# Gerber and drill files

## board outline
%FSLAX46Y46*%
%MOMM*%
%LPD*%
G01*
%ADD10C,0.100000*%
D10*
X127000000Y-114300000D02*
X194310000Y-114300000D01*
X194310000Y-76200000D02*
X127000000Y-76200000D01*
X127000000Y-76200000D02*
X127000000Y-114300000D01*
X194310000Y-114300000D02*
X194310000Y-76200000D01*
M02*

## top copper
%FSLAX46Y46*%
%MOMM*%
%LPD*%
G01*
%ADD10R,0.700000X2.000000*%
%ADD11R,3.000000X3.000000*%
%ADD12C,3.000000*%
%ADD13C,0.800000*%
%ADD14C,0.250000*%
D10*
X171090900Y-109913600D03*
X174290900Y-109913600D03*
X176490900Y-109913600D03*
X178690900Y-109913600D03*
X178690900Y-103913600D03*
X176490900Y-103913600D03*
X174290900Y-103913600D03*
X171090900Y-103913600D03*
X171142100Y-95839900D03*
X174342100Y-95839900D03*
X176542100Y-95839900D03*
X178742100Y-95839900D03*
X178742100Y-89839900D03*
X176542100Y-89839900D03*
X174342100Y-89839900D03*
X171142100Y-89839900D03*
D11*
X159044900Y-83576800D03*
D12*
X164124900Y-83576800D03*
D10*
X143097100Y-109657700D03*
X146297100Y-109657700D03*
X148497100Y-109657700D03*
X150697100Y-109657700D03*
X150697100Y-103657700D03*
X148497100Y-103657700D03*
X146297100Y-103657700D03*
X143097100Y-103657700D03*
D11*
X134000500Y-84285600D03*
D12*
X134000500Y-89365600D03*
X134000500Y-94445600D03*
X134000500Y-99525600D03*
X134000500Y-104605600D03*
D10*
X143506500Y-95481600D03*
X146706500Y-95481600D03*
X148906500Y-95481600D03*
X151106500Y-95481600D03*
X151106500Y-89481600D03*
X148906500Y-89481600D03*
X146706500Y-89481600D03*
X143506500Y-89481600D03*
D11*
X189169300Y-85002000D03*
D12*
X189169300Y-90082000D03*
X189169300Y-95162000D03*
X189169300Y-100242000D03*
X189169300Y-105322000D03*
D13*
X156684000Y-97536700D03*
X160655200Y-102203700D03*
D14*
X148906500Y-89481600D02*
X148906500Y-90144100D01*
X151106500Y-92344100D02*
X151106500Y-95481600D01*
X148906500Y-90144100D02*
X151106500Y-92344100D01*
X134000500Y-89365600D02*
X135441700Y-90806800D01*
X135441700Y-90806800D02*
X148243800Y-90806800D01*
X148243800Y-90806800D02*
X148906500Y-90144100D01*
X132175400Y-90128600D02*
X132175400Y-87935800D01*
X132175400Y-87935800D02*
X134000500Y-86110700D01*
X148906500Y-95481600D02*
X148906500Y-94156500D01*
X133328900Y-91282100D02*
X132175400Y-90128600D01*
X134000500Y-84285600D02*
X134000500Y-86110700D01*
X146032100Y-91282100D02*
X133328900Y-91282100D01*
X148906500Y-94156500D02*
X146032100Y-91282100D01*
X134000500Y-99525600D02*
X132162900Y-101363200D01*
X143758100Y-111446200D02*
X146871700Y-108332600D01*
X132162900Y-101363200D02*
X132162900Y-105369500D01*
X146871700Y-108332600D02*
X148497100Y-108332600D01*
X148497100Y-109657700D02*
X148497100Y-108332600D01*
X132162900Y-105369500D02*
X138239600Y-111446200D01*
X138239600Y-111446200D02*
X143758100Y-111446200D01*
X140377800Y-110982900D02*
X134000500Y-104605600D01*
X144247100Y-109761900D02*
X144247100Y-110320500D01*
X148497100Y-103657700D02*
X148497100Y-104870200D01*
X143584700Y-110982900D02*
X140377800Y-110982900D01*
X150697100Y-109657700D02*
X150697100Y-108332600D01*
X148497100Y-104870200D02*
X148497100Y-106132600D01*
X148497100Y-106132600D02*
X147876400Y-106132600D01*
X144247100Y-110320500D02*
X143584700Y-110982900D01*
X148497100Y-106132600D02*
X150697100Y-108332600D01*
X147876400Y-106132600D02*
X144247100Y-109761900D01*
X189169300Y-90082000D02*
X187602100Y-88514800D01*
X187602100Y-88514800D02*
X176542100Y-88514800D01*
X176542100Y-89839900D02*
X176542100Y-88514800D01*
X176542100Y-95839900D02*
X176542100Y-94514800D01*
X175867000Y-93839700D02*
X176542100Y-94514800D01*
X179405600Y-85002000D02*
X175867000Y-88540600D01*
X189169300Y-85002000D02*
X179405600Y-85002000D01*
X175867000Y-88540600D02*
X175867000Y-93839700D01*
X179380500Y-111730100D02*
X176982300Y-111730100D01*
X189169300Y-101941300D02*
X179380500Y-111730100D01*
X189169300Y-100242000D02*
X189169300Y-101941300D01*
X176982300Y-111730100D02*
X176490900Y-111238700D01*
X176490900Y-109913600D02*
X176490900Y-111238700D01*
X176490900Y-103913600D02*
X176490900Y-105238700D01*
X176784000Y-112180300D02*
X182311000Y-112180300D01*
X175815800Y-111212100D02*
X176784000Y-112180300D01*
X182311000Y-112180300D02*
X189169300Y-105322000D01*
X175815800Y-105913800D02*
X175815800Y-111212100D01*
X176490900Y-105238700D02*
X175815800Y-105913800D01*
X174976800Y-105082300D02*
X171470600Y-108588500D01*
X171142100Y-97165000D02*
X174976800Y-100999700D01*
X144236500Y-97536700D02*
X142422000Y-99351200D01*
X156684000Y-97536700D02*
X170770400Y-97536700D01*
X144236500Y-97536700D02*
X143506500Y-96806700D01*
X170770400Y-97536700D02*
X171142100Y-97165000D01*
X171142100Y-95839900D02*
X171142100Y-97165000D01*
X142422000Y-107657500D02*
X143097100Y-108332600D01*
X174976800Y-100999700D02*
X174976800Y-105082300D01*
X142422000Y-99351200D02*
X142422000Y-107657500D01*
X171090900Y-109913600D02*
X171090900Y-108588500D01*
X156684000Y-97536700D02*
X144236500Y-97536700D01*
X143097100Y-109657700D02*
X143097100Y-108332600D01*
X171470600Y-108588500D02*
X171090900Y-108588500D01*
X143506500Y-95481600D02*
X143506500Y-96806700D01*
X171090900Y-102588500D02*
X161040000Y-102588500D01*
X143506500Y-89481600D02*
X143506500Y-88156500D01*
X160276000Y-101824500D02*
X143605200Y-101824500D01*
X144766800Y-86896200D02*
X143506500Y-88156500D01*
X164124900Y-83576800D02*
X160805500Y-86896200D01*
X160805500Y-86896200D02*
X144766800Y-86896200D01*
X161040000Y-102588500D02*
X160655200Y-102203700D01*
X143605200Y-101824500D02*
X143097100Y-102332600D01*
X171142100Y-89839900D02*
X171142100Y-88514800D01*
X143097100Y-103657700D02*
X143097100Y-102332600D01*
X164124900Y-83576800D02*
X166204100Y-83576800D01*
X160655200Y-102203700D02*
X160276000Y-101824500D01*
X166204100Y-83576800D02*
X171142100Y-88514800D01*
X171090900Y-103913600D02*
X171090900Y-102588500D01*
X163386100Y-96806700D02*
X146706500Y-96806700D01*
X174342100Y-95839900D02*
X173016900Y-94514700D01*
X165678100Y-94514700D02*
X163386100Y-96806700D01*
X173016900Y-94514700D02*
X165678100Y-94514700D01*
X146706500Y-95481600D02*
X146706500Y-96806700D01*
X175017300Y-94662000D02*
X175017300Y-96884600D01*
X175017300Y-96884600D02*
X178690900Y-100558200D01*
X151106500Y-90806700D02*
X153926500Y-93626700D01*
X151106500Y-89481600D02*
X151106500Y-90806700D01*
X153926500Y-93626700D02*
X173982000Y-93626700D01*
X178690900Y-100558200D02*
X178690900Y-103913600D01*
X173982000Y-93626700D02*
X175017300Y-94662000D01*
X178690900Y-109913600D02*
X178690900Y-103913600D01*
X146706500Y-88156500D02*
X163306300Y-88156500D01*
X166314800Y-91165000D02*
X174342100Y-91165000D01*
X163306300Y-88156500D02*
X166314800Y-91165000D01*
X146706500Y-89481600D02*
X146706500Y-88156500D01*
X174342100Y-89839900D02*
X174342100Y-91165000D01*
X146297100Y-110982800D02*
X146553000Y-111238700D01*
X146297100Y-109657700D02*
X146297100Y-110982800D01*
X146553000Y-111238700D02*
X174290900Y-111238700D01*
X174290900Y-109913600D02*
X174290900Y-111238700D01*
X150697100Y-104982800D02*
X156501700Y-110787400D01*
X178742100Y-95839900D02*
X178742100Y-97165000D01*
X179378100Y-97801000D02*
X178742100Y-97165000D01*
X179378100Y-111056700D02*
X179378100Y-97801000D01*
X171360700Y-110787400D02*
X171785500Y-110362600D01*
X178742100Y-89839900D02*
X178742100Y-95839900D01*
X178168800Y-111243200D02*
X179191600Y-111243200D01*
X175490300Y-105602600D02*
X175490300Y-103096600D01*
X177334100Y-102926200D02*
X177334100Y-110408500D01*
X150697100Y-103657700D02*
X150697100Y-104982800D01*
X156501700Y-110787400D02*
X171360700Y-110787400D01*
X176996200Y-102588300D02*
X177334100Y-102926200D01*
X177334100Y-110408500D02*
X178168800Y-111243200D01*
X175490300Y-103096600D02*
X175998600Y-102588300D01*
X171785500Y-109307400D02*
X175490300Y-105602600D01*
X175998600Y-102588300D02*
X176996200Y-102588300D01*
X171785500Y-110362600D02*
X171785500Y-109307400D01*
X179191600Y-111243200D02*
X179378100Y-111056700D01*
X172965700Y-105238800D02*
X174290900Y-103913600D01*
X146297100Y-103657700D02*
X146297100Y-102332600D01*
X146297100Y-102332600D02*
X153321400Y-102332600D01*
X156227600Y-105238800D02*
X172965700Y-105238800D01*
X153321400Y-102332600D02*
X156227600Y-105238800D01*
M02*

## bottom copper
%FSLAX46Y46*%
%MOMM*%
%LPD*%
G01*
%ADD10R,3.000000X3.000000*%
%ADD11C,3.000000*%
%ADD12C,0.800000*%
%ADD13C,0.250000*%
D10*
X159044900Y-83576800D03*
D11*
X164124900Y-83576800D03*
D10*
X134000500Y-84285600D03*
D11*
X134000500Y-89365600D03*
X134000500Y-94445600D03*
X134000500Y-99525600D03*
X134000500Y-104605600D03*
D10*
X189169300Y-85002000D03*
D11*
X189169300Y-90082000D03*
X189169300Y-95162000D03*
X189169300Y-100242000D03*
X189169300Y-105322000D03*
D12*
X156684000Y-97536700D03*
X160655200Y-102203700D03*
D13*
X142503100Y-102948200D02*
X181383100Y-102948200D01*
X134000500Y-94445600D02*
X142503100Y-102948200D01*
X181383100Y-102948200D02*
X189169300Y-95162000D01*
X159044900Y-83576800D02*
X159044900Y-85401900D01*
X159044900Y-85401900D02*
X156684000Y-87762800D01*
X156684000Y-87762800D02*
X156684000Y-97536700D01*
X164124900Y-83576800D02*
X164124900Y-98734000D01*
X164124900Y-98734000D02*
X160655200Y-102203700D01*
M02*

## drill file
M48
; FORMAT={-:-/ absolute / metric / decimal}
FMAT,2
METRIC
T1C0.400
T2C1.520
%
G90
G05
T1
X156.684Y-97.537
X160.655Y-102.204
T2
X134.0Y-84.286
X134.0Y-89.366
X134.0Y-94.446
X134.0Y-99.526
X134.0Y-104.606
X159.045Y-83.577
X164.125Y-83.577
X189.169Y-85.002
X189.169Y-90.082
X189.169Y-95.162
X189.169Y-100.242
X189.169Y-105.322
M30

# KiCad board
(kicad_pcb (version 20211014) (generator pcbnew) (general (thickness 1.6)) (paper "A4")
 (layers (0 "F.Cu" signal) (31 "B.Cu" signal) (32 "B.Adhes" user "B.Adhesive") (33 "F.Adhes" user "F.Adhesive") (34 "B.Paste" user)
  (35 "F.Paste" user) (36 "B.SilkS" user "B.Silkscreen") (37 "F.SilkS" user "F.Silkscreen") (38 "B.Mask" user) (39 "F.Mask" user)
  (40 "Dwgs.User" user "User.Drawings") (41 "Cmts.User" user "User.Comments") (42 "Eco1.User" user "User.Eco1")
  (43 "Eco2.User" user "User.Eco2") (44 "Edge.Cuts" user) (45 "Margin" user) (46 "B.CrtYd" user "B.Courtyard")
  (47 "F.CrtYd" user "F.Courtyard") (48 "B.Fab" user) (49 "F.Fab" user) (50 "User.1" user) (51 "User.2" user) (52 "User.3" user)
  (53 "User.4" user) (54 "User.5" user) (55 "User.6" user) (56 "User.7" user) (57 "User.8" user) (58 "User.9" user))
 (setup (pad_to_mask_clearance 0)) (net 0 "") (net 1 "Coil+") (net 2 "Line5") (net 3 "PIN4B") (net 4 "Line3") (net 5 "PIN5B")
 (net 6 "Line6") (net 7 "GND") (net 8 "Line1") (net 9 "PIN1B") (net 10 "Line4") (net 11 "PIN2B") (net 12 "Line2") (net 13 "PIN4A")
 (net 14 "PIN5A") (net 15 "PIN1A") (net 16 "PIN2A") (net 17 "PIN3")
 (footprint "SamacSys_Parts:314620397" (layer "F.Cu") (at 174.8909 106.9136)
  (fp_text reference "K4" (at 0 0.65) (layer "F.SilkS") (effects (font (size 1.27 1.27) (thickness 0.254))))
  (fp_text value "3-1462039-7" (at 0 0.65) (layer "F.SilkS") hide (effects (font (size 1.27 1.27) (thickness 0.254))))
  (pad "1" smd rect locked (at -3.8 3) (size 0.7 2) (layers "F.Cu" "F.Paste" "F.Mask") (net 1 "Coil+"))
  (pad "2" smd rect locked (at -0.6 3) (size 0.7 2) (layers "F.Cu" "F.Paste" "F.Mask") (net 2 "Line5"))
  (pad "3" smd rect locked (at 1.6 3) (size 0.7 2) (layers "F.Cu" "F.Paste" "F.Mask") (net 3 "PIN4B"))
  (pad "4" smd rect locked (at 3.8 3) (size 0.7 2) (layers "F.Cu" "F.Paste" "F.Mask") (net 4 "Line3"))
  (pad "5" smd rect locked (at 3.8 -3) (size 0.7 2) (layers "F.Cu" "F.Paste" "F.Mask") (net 4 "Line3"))
  (pad "6" smd rect locked (at 1.6 -3) (size 0.7 2) (layers "F.Cu" "F.Paste" "F.Mask") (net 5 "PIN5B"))
  (pad "7" smd rect locked (at -0.6 -3) (size 0.7 2) (layers "F.Cu" "F.Paste" "F.Mask") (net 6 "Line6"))
  (pad "8" smd rect locked (at -3.8 -3) (size 0.7 2) (layers "F.Cu" "F.Paste" "F.Mask") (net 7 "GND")))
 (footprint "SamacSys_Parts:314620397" (layer "F.Cu") (at 174.9421 92.8399)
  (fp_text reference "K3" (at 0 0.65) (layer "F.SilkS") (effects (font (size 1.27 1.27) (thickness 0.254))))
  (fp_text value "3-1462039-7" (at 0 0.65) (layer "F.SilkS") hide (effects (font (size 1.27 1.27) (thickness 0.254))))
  (pad "1" smd rect locked (at -3.8 3) (size 0.7 2) (layers "F.Cu" "F.Paste" "F.Mask") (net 1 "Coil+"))
  (pad "2" smd rect locked (at -0.6 3) (size 0.7 2) (layers "F.Cu" "F.Paste" "F.Mask") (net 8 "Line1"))
  (pad "3" smd rect locked (at 1.6 3) (size 0.7 2) (layers "F.Cu" "F.Paste" "F.Mask") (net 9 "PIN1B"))
  (pad "4" smd rect locked (at 3.8 3) (size 0.7 2) (layers "F.Cu" "F.Paste" "F.Mask") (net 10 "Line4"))
  (pad "5" smd rect locked (at 3.8 -3) (size 0.7 2) (layers "F.Cu" "F.Paste" "F.Mask") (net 10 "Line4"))
  (pad "6" smd rect locked (at 1.6 -3) (size 0.7 2) (layers "F.Cu" "F.Paste" "F.Mask") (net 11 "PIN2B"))
  (pad "7" smd rect locked (at -0.6 -3) (size 0.7 2) (layers "F.Cu" "F.Paste" "F.Mask") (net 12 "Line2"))
  (pad "8" smd rect locked (at -3.8 -3) (size 0.7 2) (layers "F.Cu" "F.Paste" "F.Mask") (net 7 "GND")))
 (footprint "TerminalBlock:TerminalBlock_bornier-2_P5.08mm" (layer "F.Cu") (at 159.0449 83.5768)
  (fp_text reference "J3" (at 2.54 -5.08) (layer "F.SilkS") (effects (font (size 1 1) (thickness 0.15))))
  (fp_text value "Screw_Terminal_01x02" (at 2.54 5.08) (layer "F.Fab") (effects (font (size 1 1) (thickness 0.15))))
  (pad "1" thru_hole rect locked (at 0 0) (size 3 3) (drill 1.52) (layers *.Cu *.Mask) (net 1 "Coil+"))
  (pad "2" thru_hole circle locked (at 5.08 0) (size 3 3) (drill 1.52) (layers *.Cu *.Mask) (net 7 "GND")))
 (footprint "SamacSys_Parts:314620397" (layer "F.Cu") (at 146.8971 106.6577)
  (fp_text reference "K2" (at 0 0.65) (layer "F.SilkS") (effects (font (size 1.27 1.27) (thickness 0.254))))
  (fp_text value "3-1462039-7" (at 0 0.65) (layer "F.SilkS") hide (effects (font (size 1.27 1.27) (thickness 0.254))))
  (pad "1" smd rect locked (at -3.8 3) (size 0.7 2) (layers "F.Cu" "F.Paste" "F.Mask") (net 1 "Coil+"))
  (pad "2" smd rect locked (at -0.6 3) (size 0.7 2) (layers "F.Cu" "F.Paste" "F.Mask") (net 2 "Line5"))
  (pad "3" smd rect locked (at 1.6 3) (size 0.7 2) (layers "F.Cu" "F.Paste" "F.Mask") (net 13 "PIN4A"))
  (pad "4" smd rect locked (at 3.8 3) (size 0.7 2) (layers "F.Cu" "F.Paste" "F.Mask") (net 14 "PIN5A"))
  (pad "5" smd rect locked (at 3.8 -3) (size 0.7 2) (layers "F.Cu" "F.Paste" "F.Mask") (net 10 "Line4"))
  (pad "6" smd rect locked (at 1.6 -3) (size 0.7 2) (layers "F.Cu" "F.Paste" "F.Mask") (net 14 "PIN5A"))
  (pad "7" smd rect locked (at -0.6 -3) (size 0.7 2) (layers "F.Cu" "F.Paste" "F.Mask") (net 6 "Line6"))
  (pad "8" smd rect locked (at -3.8 -3) (size 0.7 2) (layers "F.Cu" "F.Paste" "F.Mask") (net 7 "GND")))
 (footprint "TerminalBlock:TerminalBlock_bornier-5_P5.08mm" (layer "F.Cu") (at 134.0005 84.2856 -90)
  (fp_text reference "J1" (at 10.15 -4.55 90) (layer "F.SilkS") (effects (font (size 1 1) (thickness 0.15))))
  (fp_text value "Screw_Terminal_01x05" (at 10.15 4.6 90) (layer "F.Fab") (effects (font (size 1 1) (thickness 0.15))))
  (pad "1" thru_hole rect locked (at 0 0 270) (size 3 3) (drill 1.52) (layers *.Cu *.Mask) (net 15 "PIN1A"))
  (pad "2" thru_hole circle locked (at 5.08 0 270) (size 3 3) (drill 1.52) (layers *.Cu *.Mask) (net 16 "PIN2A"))
  (pad "3" thru_hole circle locked (at 10.16 0 270) (size 3 3) (drill 1.52) (layers *.Cu *.Mask) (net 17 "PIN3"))
  (pad "4" thru_hole circle locked (at 15.24 0 270) (size 3 3) (drill 1.52) (layers *.Cu *.Mask) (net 13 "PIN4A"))
  (pad "5" thru_hole circle locked (at 20.32 0 270) (size 3 3) (drill 1.52) (layers *.Cu *.Mask) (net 14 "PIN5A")))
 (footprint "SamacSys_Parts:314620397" (layer "F.Cu") (at 147.3065 92.4816)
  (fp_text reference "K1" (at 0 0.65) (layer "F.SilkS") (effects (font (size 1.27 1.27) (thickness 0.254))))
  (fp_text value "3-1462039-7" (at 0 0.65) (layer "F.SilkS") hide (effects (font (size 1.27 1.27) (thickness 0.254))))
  (pad "1" smd rect locked (at -3.8 3) (size 0.7 2) (layers "F.Cu" "F.Paste" "F.Mask") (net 1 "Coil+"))
  (pad "2" smd rect locked (at -0.6 3) (size 0.7 2) (layers "F.Cu" "F.Paste" "F.Mask") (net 8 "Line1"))
  (pad "3" smd rect locked (at 1.6 3) (size 0.7 2) (layers "F.Cu" "F.Paste" "F.Mask") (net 15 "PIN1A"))
  (pad "4" smd rect locked (at 3.8 3) (size 0.7 2) (layers "F.Cu" "F.Paste" "F.Mask") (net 16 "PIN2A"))
  (pad "5" smd rect locked (at 3.8 -3) (size 0.7 2) (layers "F.Cu" "F.Paste" "F.Mask") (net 4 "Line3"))
  (pad "6" smd rect locked (at 1.6 -3) (size 0.7 2) (layers "F.Cu" "F.Paste" "F.Mask") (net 16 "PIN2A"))
  (pad "7" smd rect locked (at -0.6 -3) (size 0.7 2) (layers "F.Cu" "F.Paste" "F.Mask") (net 12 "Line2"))
  (pad "8" smd rect locked (at -3.8 -3) (size 0.7 2) (layers "F.Cu" "F.Paste" "F.Mask") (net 7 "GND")))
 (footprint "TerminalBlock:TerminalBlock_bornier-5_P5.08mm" (layer "F.Cu") (at 189.1693 85.002 -90)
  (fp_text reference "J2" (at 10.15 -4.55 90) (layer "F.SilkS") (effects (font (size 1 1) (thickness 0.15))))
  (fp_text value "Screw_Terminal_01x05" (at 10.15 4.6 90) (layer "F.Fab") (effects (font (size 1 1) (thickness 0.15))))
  (pad "1" thru_hole rect locked (at 0 0 270) (size 3 3) (drill 1.52) (layers *.Cu *.Mask) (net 9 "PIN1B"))
  (pad "2" thru_hole circle locked (at 5.08 0 270) (size 3 3) (drill 1.52) (layers *.Cu *.Mask) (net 11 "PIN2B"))
  (pad "3" thru_hole circle locked (at 10.16 0 270) (size 3 3) (drill 1.52) (layers *.Cu *.Mask) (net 17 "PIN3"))
  (pad "4" thru_hole circle locked (at 15.24 0 270) (size 3 3) (drill 1.52) (layers *.Cu *.Mask) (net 3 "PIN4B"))
  (pad "5" thru_hole circle locked (at 20.32 0 270) (size 3 3) (drill 1.52) (layers *.Cu *.Mask) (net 5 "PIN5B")))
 (gr_line (start 127 114.3) (end 194.31 114.3) (layer "Edge.Cuts") (width 0.1))
 (gr_line (start 194.31 76.2) (end 127 76.2) (layer "Edge.Cuts") (width 0.1))
 (gr_line (start 127 76.2) (end 127 114.3) (layer "Edge.Cuts") (width 0.1))
 (gr_line (start 194.31 114.3) (end 194.31 76.2) (layer "Edge.Cuts") (width 0.1))
 (segment (start 148.9065 89.4816) (end 148.9065 90.1441) (width 0.25) (layer "F.Cu") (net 16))
 (segment (start 151.1065 92.3441) (end 151.1065 95.4816) (width 0.25) (layer "F.Cu") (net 16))
 (segment (start 148.9065 90.1441) (end 151.1065 92.3441) (width 0.25) (layer "F.Cu") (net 16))
 (segment (start 134.0005 89.3656) (end 135.4417 90.8068) (width 0.25) (layer "F.Cu") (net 16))
 (segment (start 135.4417 90.8068) (end 148.2438 90.8068) (width 0.25) (layer "F.Cu") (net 16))
 (segment (start 148.2438 90.8068) (end 148.9065 90.1441) (width 0.25) (layer "F.Cu") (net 16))
 (segment (start 142.5031 102.9482) (end 181.3831 102.9482) (width 0.25) (layer "B.Cu") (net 17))
 (segment (start 134.0005 94.4456) (end 142.5031 102.9482) (width 0.25) (layer "B.Cu") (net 17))
 (segment (start 181.3831 102.9482) (end 189.1693 95.162) (width 0.25) (layer "B.Cu") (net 17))
 (segment (start 132.1754 90.1286) (end 132.1754 87.9358) (width 0.25) (layer "F.Cu") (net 15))
 (segment (start 132.1754 87.9358) (end 134.0005 86.1107) (width 0.25) (layer "F.Cu") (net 15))
 (segment (start 148.9065 95.4816) (end 148.9065 94.1565) (width 0.25) (layer "F.Cu") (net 15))
 (segment (start 133.3289 91.2821) (end 132.1754 90.1286) (width 0.25) (layer "F.Cu") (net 15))
 (segment (start 134.0005 84.2856) (end 134.0005 86.1107) (width 0.25) (layer "F.Cu") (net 15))
 (segment (start 146.0321 91.2821) (end 133.3289 91.2821) (width 0.25) (layer "F.Cu") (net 15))
 (segment (start 148.9065 94.1565) (end 146.0321 91.2821) (width 0.25) (layer "F.Cu") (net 15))
 (segment (start 134.0005 99.5256) (end 132.1629 101.3632) (width 0.25) (layer "F.Cu") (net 13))
 (segment (start 143.7581 111.4462) (end 146.8717 108.3326) (width 0.25) (layer "F.Cu") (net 13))
 (segment (start 132.1629 101.3632) (end 132.1629 105.3695) (width 0.25) (layer "F.Cu") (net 13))
 (segment (start 146.8717 108.3326) (end 148.4971 108.3326) (width 0.25) (layer "F.Cu") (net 13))
 (segment (start 148.4971 109.6577) (end 148.4971 108.3326) (width 0.25) (layer "F.Cu") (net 13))
 (segment (start 132.1629 105.3695) (end 138.2396 111.4462) (width 0.25) (layer "F.Cu") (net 13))
 (segment (start 138.2396 111.4462) (end 143.7581 111.4462) (width 0.25) (layer "F.Cu") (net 13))
 (segment (start 140.3778 110.9829) (end 134.0005 104.6056) (width 0.25) (layer "F.Cu") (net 14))
 (segment (start 144.2471 109.7619) (end 144.2471 110.3205) (width 0.25) (layer "F.Cu") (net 14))
 (segment (start 148.4971 103.6577) (end 148.4971 104.8702) (width 0.25) (layer "F.Cu") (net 14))
 (segment (start 143.5847 110.9829) (end 140.3778 110.9829) (width 0.25) (layer "F.Cu") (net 14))
 (segment (start 150.6971 109.6577) (end 150.6971 108.3326) (width 0.25) (layer "F.Cu") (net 14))
 (segment (start 148.4971 104.8702) (end 148.4971 106.1326) (width 0.25) (layer "F.Cu") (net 14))
 (segment (start 148.4971 106.1326) (end 147.8764 106.1326) (width 0.25) (layer "F.Cu") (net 14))
 (segment (start 144.2471 110.3205) (end 143.5847 110.9829) (width 0.25) (layer "F.Cu") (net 14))
 (segment (start 148.4971 106.1326) (end 150.6971 108.3326) (width 0.25) (layer "F.Cu") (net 14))
 (segment (start 147.8764 106.1326) (end 144.2471 109.7619) (width 0.25) (layer "F.Cu") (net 14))
 (segment (start 189.1693 90.082) (end 187.6021 88.5148) (width 0.25) (layer "F.Cu") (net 11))
 (segment (start 187.6021 88.5148) (end 176.5421 88.5148) (width 0.25) (layer "F.Cu") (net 11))
 (segment (start 176.5421 89.8399) (end 176.5421 88.5148) (width 0.25) (layer "F.Cu") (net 11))
 (segment (start 176.5421 95.8399) (end 176.5421 94.5148) (width 0.25) (layer "F.Cu") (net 9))
 (segment (start 175.867 93.8397) (end 176.5421 94.5148) (width 0.25) (layer "F.Cu") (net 9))
 (segment (start 179.4056 85.002) (end 175.867 88.5406) (width 0.25) (layer "F.Cu") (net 9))
 (segment (start 189.1693 85.002) (end 179.4056 85.002) (width 0.25) (layer "F.Cu") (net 9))
 (segment (start 175.867 88.5406) (end 175.867 93.8397) (width 0.25) (layer "F.Cu") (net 9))
 (segment (start 179.3805 111.7301) (end 176.9823 111.7301) (width 0.25) (layer "F.Cu") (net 3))
 (segment (start 189.1693 101.9413) (end 179.3805 111.7301) (width 0.25) (layer "F.Cu") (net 3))
 (segment (start 189.1693 100.242) (end 189.1693 101.9413) (width 0.25) (layer "F.Cu") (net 3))
 (segment (start 176.9823 111.7301) (end 176.4909 111.2387) (width 0.25) (layer "F.Cu") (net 3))
 (segment (start 176.4909 109.9136) (end 176.4909 111.2387) (width 0.25) (layer "F.Cu") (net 3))
 (segment (start 176.4909 103.9136) (end 176.4909 105.2387) (width 0.25) (layer "F.Cu") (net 5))
 (segment (start 176.784 112.1803) (end 182.311 112.1803) (width 0.25) (layer "F.Cu") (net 5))
 (segment (start 175.8158 111.2121) (end 176.784 112.1803) (width 0.25) (layer "F.Cu") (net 5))
 (segment (start 182.311 112.1803) (end 189.1693 105.322) (width 0.25) (layer "F.Cu") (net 5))
 (segment (start 175.8158 105.9138) (end 175.8158 111.2121) (width 0.25) (layer "F.Cu") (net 5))
 (segment (start 176.4909 105.2387) (end 175.8158 105.9138) (width 0.25) (layer "F.Cu") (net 5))
 (segment (start 174.9768 105.0823) (end 171.4706 108.5885) (width 0.25) (layer "F.Cu") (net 1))
 (segment (start 171.1421 97.165) (end 174.9768 100.9997) (width 0.25) (layer "F.Cu") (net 1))
 (segment (start 144.2365 97.5367) (end 142.422 99.3512) (width 0.25) (layer "F.Cu") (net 1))
 (segment (start 156.684 97.5367) (end 170.7704 97.5367) (width 0.25) (layer "F.Cu") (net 1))
 (segment (start 144.2365 97.5367) (end 143.5065 96.8067) (width 0.25) (layer "F.Cu") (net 1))
 (segment (start 170.7704 97.5367) (end 171.1421 97.165) (width 0.25) (layer "F.Cu") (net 1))
 (segment (start 171.1421 95.8399) (end 171.1421 97.165) (width 0.25) (layer "F.Cu") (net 1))
 (segment (start 142.422 107.6575) (end 143.0971 108.3326) (width 0.25) (layer "F.Cu") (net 1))
 (segment (start 174.9768 100.9997) (end 174.9768 105.0823) (width 0.25) (layer "F.Cu") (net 1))
 (segment (start 142.422 99.3512) (end 142.422 107.6575) (width 0.25) (layer "F.Cu") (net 1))
 (segment (start 171.0909 109.9136) (end 171.0909 108.5885) (width 0.25) (layer "F.Cu") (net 1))
 (segment (start 156.684 97.5367) (end 144.2365 97.5367) (width 0.25) (layer "F.Cu") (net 1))
 (segment (start 143.0971 109.6577) (end 143.0971 108.3326) (width 0.25) (layer "F.Cu") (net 1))
 (segment (start 171.4706 108.5885) (end 171.0909 108.5885) (width 0.25) (layer "F.Cu") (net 1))
 (segment (start 143.5065 95.4816) (end 143.5065 96.8067) (width 0.25) (layer "F.Cu") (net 1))
 (via (at 156.684 97.5367) (size 0.8) (drill 0.4) (layers "F.Cu" "B.Cu") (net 1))
 (segment (start 159.0449 83.5768) (end 159.0449 85.4019) (width 0.25) (layer "B.Cu") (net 1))
 (segment (start 159.0449 85.4019) (end 156.684 87.7628) (width 0.25) (layer "B.Cu") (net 1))
 (segment (start 156.684 87.7628) (end 156.684 97.5367) (width 0.25) (layer "B.Cu") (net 1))
 (segment (start 171.0909 102.5885) (end 161.04 102.5885) (width 0.25) (layer "F.Cu") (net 7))
 (segment (start 143.5065 89.4816) (end 143.5065 88.1565) (width 0.25) (layer "F.Cu") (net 7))
 (segment (start 160.276 101.8245) (end 143.6052 101.8245) (width 0.25) (layer "F.Cu") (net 7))
 (segment (start 144.7668 86.8962) (end 143.5065 88.1565) (width 0.25) (layer "F.Cu") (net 7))
 (segment (start 164.1249 83.5768) (end 160.8055 86.8962) (width 0.25) (layer "F.Cu") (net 7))
 (segment (start 160.8055 86.8962) (end 144.7668 86.8962) (width 0.25) (layer "F.Cu") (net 7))
 (segment (start 161.04 102.5885) (end 160.6552 102.2037) (width 0.25) (layer "F.Cu") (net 7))
 (segment (start 143.6052 101.8245) (end 143.0971 102.3326) (width 0.25) (layer "F.Cu") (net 7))
 (segment (start 171.1421 89.8399) (end 171.1421 88.5148) (width 0.25) (layer "F.Cu") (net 7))
 (segment (start 143.0971 103.6577) (end 143.0971 102.3326) (width 0.25) (layer "F.Cu") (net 7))
 (segment (start 164.1249 83.5768) (end 166.2041 83.5768) (width 0.25) (layer "F.Cu") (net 7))
 (segment (start 160.6552 102.2037) (end 160.276 101.8245) (width 0.25) (layer "F.Cu") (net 7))
 (segment (start 166.2041 83.5768) (end 171.1421 88.5148) (width 0.25) (layer "F.Cu") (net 7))
 (segment (start 171.0909 103.9136) (end 171.0909 102.5885) (width 0.25) (layer "F.Cu") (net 7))
 (via (at 160.6552 102.2037) (size 0.8) (drill 0.4) (layers "F.Cu" "B.Cu") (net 7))
 (segment (start 164.1249 83.5768) (end 164.1249 98.734) (width 0.25) (layer "B.Cu") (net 7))
 (segment (start 164.1249 98.734) (end 160.6552 102.2037) (width 0.25) (layer "B.Cu") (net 7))
 (segment (start 163.3861 96.8067) (end 146.7065 96.8067) (width 0.25) (layer "F.Cu") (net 8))
 (segment (start 174.3421 95.8399) (end 173.0169 94.5147) (width 0.25) (layer "F.Cu") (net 8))
 (segment (start 165.6781 94.5147) (end 163.3861 96.8067) (width 0.25) (layer "F.Cu") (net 8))
 (segment (start 173.0169 94.5147) (end 165.6781 94.5147) (width 0.25) (layer "F.Cu") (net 8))
 (segment (start 146.7065 95.4816) (end 146.7065 96.8067) (width 0.25) (layer "F.Cu") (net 8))
 (segment (start 175.0173 94.662) (end 175.0173 96.8846) (width 0.25) (layer "F.Cu") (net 4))
 (segment (start 175.0173 96.8846) (end 178.6909 100.5582) (width 0.25) (layer "F.Cu") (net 4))
 (segment (start 151.1065 90.8067) (end 153.9265 93.6267) (width 0.25) (layer "F.Cu") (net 4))
 (segment (start 151.1065 89.4816) (end 151.1065 90.8067) (width 0.25) (layer "F.Cu") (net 4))
 (segment (start 153.9265 93.6267) (end 173.982 93.6267) (width 0.25) (layer "F.Cu") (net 4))
 (segment (start 178.6909 100.5582) (end 178.6909 103.9136) (width 0.25) (layer "F.Cu") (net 4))
 (segment (start 173.982 93.6267) (end 175.0173 94.662) (width 0.25) (layer "F.Cu") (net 4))
 (segment (start 178.6909 109.9136) (end 178.6909 103.9136) (width 0.25) (layer "F.Cu") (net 4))
 (segment (start 146.7065 88.1565) (end 163.3063 88.1565) (width 0.25) (layer "F.Cu") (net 12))
 (segment (start 166.3148 91.165) (end 174.3421 91.165) (width 0.25) (layer "F.Cu") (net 12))
 (segment (start 163.3063 88.1565) (end 166.3148 91.165) (width 0.25) (layer "F.Cu") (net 12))
 (segment (start 146.7065 89.4816) (end 146.7065 88.1565) (width 0.25) (layer "F.Cu") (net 12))
 (segment (start 174.3421 89.8399) (end 174.3421 91.165) (width 0.25) (layer "F.Cu") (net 12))
 (segment (start 146.2971 110.9828) (end 146.553 111.2387) (width 0.25) (layer "F.Cu") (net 2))
 (segment (start 146.2971 109.6577) (end 146.2971 110.9828) (width 0.25) (layer "F.Cu") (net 2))
 (segment (start 146.553 111.2387) (end 174.2909 111.2387) (width 0.25) (layer "F.Cu") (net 2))
 (segment (start 174.2909 109.9136) (end 174.2909 111.2387) (width 0.25) (layer "F.Cu") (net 2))
 (segment (start 150.6971 104.9828) (end 156.5017 110.7874) (width 0.25) (layer "F.Cu") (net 10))
 (segment (start 178.7421 95.8399) (end 178.7421 97.165) (width 0.25) (layer "F.Cu") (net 10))
 (segment (start 179.3781 97.801) (end 178.7421 97.165) (width 0.25) (layer "F.Cu") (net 10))
 (segment (start 179.3781 111.0567) (end 179.3781 97.801) (width 0.25) (layer "F.Cu") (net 10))
 (segment (start 171.3607 110.7874) (end 171.7855 110.3626) (width 0.25) (layer "F.Cu") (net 10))
 (segment (start 178.7421 89.8399) (end 178.7421 95.8399) (width 0.25) (layer "F.Cu") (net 10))
 (segment (start 178.1688 111.2432) (end 179.1916 111.2432) (width 0.25) (layer "F.Cu") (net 10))
 (segment (start 175.4903 105.6026) (end 175.4903 103.0966) (width 0.25) (layer "F.Cu") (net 10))
 (segment (start 177.3341 102.9262) (end 177.3341 110.4085) (width 0.25) (layer "F.Cu") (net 10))
 (segment (start 150.6971 103.6577) (end 150.6971 104.9828) (width 0.25) (layer "F.Cu") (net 10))
 (segment (start 156.5017 110.7874) (end 171.3607 110.7874) (width 0.25) (layer "F.Cu") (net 10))
 (segment (start 176.9962 102.5883) (end 177.3341 102.9262) (width 0.25) (layer "F.Cu") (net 10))
 (segment (start 177.3341 110.4085) (end 178.1688 111.2432) (width 0.25) (layer "F.Cu") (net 10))
 (segment (start 175.4903 103.0966) (end 175.9986 102.5883) (width 0.25) (layer "F.Cu") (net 10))
 (segment (start 171.7855 109.3074) (end 175.4903 105.6026) (width 0.25) (layer "F.Cu") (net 10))
 (segment (start 175.9986 102.5883) (end 176.9962 102.5883) (width 0.25) (layer "F.Cu") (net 10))
 (segment (start 171.7855 110.3626) (end 171.7855 109.3074) (width 0.25) (layer "F.Cu") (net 10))
 (segment (start 179.1916 111.2432) (end 179.3781 111.0567) (width 0.25) (layer "F.Cu") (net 10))
 (segment (start 172.9657 105.2388) (end 174.2909 103.9136) (width 0.25) (layer "F.Cu") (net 6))
 (segment (start 146.2971 103.6577) (end 146.2971 102.3326) (width 0.25) (layer "F.Cu") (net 6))
 (segment (start 146.2971 102.3326) (end 153.3214 102.3326) (width 0.25) (layer "F.Cu") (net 6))
 (segment (start 156.2276 105.2388) (end 172.9657 105.2388) (width 0.25) (layer "F.Cu") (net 6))
 (segment (start 153.3214 102.3326) (end 156.2276 105.2388) (width 0.25) (layer "F.Cu") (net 6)))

